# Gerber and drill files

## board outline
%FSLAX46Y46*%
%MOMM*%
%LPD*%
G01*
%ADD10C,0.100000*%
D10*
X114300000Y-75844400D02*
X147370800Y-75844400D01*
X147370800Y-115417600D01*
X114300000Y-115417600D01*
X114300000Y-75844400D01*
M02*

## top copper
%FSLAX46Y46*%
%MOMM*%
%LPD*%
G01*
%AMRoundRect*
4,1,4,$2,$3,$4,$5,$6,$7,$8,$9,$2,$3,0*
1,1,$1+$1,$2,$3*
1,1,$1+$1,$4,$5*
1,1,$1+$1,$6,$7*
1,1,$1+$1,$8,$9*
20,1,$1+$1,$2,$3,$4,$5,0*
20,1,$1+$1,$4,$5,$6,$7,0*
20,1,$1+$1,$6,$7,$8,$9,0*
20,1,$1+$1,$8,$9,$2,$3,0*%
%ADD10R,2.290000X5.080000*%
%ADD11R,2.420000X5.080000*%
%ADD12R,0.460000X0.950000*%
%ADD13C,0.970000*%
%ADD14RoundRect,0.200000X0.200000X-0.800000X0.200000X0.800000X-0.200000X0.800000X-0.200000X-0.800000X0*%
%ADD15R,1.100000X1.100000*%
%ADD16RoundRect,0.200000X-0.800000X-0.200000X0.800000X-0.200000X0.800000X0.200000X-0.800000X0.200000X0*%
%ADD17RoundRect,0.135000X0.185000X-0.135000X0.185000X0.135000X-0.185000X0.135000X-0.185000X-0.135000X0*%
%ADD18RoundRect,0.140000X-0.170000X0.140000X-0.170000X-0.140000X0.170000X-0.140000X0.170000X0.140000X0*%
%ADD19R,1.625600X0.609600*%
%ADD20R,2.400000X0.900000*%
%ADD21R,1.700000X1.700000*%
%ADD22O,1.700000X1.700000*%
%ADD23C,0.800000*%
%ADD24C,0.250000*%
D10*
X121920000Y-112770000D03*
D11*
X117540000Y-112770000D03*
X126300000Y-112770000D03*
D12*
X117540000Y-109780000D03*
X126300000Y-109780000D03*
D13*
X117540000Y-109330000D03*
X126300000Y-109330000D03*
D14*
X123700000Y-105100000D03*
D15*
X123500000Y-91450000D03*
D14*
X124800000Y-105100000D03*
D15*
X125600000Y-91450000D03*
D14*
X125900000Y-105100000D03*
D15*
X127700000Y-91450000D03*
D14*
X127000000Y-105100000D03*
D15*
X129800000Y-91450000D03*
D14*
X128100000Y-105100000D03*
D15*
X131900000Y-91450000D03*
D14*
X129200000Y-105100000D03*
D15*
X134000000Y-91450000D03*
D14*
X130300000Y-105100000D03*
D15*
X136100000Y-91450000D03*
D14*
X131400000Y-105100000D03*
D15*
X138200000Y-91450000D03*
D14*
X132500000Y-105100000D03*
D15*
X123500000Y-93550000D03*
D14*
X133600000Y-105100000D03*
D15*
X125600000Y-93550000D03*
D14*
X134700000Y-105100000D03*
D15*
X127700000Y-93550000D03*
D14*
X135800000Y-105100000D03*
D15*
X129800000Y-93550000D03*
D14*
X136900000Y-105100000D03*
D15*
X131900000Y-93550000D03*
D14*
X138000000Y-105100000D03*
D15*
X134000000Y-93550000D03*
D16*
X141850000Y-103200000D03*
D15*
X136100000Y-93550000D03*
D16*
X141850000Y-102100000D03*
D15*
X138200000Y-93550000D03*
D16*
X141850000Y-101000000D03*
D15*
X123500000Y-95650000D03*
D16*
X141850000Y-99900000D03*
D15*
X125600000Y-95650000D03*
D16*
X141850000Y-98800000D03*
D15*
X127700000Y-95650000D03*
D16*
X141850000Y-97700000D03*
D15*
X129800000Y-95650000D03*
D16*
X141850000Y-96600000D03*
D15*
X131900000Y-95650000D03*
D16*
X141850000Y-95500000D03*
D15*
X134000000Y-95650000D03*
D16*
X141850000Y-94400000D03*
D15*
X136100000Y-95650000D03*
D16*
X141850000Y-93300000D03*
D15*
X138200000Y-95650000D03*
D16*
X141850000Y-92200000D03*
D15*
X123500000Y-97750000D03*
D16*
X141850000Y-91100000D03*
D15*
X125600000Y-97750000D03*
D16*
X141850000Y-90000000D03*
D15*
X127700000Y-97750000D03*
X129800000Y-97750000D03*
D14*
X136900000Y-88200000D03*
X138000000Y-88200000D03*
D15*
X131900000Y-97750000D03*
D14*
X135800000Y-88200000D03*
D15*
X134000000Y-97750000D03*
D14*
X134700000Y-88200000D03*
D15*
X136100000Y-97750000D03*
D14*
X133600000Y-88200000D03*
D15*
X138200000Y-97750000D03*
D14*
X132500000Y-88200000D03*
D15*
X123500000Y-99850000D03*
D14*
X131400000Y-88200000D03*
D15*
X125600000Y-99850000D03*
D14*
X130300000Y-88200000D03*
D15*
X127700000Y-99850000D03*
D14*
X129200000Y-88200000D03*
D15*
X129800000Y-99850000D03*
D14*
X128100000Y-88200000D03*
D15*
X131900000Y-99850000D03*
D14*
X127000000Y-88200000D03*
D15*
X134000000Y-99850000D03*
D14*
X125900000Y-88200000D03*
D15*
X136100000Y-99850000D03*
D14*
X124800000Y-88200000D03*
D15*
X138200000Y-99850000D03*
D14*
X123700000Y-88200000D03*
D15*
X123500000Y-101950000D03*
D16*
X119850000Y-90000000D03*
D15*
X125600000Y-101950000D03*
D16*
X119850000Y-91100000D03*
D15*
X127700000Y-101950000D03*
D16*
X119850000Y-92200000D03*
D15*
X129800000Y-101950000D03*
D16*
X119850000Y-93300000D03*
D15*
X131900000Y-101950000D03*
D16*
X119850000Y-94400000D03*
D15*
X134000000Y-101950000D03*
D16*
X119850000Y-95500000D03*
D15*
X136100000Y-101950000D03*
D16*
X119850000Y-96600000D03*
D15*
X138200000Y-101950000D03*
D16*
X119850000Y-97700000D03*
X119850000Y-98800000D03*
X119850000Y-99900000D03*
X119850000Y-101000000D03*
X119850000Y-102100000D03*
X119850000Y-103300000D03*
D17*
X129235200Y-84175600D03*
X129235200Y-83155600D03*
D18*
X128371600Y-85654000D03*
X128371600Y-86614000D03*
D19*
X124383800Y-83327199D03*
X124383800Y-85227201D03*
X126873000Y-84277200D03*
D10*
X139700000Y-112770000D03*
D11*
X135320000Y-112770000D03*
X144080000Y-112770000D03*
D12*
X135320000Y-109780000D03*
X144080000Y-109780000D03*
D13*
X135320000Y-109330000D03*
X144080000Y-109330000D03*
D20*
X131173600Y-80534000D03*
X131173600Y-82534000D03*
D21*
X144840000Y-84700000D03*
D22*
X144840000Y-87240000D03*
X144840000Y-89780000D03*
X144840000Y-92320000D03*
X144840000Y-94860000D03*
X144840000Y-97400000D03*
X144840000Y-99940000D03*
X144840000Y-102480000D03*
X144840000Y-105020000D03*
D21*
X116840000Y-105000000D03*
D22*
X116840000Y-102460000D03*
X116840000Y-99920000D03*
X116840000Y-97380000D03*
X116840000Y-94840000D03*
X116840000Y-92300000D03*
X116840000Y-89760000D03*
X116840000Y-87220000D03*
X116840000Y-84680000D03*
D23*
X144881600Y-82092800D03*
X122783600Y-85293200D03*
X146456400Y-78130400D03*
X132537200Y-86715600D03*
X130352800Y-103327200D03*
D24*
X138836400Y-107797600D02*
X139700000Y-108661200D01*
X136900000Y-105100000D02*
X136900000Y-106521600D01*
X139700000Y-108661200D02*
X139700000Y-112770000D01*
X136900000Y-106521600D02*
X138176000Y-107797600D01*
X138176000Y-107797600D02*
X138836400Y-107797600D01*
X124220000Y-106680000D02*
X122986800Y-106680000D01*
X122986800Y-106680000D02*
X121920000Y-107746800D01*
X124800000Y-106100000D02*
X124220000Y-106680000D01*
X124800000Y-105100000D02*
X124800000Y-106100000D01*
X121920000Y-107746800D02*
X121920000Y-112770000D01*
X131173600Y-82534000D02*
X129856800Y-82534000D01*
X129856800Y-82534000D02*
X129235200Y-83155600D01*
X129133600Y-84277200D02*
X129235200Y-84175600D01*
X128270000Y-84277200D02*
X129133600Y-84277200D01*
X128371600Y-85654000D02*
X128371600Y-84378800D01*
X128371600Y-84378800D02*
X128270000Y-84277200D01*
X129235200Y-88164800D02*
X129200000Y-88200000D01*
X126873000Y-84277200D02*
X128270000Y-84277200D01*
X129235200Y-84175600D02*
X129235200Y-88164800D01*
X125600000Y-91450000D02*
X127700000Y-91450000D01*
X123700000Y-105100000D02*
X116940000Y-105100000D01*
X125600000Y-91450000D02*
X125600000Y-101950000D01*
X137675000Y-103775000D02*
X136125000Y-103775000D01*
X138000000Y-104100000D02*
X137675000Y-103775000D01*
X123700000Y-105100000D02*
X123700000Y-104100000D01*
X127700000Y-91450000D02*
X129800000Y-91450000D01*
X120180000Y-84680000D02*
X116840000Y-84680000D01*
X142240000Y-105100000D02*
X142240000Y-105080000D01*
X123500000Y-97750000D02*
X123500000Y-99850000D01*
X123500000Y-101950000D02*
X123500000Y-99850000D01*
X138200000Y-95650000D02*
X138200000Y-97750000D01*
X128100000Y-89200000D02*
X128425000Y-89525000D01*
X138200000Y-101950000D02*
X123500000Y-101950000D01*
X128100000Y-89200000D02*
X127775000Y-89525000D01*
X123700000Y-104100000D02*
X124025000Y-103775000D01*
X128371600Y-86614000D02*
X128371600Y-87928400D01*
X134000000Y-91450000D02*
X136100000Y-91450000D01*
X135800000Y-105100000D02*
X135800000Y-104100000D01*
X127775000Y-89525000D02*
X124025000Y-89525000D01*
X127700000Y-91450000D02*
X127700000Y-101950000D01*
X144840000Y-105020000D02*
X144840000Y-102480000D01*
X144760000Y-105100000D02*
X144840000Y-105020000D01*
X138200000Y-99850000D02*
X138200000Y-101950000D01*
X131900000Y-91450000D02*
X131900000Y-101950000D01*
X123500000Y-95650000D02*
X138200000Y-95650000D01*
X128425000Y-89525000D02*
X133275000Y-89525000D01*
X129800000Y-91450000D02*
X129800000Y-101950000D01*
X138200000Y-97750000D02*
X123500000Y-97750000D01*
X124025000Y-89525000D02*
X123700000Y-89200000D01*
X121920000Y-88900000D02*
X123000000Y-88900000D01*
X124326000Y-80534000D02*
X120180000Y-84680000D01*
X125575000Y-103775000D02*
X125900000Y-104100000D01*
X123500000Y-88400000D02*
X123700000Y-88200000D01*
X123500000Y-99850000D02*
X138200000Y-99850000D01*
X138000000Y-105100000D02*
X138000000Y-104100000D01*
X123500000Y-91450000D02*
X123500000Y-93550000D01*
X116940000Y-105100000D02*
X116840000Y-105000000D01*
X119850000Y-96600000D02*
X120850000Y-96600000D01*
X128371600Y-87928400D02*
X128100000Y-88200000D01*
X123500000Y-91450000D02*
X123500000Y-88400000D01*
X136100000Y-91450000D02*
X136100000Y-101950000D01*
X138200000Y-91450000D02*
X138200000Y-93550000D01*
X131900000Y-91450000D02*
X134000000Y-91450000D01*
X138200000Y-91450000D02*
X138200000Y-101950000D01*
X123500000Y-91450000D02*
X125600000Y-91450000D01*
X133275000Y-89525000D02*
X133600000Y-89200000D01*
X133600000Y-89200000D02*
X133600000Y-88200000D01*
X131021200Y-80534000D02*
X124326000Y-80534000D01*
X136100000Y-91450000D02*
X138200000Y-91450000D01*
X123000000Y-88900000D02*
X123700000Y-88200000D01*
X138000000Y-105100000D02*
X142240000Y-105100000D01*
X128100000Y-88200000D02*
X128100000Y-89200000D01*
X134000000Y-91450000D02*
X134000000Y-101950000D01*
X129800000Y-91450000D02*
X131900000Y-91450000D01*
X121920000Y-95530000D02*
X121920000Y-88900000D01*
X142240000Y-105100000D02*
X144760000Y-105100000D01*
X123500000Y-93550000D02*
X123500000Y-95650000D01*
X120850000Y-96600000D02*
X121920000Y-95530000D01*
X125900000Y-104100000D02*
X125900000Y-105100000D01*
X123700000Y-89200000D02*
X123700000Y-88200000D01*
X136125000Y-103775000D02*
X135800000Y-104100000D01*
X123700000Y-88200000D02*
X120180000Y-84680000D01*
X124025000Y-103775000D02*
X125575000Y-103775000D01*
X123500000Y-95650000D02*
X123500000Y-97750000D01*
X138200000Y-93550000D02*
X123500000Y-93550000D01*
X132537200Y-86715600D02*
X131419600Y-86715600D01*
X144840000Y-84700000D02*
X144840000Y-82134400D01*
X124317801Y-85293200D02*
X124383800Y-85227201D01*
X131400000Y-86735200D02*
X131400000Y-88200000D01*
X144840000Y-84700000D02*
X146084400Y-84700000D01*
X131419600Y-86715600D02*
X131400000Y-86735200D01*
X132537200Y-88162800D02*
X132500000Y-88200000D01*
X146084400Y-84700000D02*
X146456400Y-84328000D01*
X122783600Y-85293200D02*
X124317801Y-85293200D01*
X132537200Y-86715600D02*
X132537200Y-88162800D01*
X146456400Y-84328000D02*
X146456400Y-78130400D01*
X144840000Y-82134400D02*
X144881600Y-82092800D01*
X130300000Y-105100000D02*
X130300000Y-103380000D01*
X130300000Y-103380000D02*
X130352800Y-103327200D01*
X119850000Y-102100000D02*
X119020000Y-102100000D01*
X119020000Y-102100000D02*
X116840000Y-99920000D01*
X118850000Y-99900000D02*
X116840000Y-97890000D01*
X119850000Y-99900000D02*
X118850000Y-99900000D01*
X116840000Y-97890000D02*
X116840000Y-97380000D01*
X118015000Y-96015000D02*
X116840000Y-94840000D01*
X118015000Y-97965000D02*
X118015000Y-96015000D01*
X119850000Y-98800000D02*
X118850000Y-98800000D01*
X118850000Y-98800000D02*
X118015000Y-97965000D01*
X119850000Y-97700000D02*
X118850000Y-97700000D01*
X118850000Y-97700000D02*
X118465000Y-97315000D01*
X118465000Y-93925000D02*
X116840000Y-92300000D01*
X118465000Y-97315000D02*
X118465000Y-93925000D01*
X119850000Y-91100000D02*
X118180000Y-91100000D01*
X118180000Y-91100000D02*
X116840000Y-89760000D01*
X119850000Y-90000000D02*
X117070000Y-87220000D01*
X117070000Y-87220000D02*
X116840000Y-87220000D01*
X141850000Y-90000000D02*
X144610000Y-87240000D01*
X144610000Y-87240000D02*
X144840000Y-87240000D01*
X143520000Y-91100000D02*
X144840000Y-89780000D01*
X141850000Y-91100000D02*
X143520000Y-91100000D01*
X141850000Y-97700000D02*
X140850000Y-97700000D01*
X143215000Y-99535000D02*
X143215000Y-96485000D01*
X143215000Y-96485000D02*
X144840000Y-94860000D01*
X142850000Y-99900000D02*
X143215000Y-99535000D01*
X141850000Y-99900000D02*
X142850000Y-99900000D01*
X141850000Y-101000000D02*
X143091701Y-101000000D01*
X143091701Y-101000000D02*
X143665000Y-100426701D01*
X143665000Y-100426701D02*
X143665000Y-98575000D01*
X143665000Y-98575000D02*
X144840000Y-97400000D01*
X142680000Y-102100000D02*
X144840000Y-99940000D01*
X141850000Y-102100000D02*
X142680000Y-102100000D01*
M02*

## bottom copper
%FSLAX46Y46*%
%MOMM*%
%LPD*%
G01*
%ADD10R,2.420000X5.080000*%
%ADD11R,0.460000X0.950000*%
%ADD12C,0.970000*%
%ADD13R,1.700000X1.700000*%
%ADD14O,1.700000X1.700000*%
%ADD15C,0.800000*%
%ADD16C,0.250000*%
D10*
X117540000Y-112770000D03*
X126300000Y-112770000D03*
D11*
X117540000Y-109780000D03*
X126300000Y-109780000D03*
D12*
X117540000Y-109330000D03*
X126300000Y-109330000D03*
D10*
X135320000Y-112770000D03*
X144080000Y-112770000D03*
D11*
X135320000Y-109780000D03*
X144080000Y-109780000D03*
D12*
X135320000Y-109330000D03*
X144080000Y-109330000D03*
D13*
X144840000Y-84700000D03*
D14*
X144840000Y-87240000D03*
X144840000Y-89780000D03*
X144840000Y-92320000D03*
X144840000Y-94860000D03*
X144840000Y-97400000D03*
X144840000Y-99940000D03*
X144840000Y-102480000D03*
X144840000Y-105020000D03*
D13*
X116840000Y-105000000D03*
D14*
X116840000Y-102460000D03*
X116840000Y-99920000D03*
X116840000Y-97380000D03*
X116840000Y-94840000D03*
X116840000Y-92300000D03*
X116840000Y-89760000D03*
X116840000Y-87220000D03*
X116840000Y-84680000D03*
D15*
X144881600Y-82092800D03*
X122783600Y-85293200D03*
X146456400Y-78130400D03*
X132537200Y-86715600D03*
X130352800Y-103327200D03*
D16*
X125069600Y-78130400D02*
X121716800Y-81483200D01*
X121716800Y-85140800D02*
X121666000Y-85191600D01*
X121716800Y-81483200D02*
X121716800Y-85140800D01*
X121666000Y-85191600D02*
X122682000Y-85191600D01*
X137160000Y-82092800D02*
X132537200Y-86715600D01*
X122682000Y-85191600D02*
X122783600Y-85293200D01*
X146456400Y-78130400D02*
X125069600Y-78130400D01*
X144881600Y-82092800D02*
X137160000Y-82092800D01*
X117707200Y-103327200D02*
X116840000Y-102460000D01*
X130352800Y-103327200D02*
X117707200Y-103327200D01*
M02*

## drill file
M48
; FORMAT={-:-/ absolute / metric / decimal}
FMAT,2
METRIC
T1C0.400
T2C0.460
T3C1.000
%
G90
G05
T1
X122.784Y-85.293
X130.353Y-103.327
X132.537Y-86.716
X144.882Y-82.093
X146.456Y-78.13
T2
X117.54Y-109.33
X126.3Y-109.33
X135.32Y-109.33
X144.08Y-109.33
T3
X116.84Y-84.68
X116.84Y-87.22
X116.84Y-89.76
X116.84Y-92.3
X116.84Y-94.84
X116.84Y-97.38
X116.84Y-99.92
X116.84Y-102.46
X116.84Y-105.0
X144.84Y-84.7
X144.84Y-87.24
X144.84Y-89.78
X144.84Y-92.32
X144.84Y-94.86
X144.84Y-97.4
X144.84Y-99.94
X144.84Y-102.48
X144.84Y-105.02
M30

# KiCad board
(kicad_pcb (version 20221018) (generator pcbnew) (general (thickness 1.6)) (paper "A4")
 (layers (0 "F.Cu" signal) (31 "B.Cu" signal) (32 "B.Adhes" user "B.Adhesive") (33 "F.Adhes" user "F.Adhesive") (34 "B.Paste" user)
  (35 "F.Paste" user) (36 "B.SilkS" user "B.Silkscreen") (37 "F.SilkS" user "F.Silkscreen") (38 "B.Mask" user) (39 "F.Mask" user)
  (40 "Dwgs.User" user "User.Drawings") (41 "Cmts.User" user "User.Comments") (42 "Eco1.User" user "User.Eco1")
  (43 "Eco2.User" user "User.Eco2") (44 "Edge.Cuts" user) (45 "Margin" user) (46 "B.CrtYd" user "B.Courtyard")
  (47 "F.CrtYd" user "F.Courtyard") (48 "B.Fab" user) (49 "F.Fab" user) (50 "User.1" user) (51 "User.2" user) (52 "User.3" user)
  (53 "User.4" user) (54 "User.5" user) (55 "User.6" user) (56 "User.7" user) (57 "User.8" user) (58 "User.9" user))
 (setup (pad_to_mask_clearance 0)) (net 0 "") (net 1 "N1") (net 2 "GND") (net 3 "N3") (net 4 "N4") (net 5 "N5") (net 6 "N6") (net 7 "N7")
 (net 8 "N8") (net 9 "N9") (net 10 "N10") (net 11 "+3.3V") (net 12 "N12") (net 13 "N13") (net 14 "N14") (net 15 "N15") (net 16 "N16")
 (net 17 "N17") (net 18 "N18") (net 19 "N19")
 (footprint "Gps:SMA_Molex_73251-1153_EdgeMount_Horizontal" (layer "F.Cu") (at 121.92 111.05 90)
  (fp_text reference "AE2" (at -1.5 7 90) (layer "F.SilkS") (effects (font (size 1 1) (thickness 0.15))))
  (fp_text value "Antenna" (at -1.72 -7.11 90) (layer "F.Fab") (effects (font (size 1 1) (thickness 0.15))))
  (pad "1" smd rect (at -1.72 0 90) (size 5.08 2.29) (layers "F.Cu" "F.Paste" "F.Mask") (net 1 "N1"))
  (pad "2" smd rect (at -1.72 -4.38 90) (size 5.08 2.42) (layers "F.Cu" "F.Paste" "F.Mask"))
  (pad "2" smd rect (at -1.72 -4.38 90) (size 5.08 2.42) (layers "B.Cu" "B.Paste" "B.Mask"))
  (pad "2" smd rect (at -1.72 4.38 90) (size 5.08 2.42) (layers "F.Cu" "F.Paste" "F.Mask"))
  (pad "2" smd rect (at -1.72 4.38 90) (size 5.08 2.42) (layers "B.Cu" "B.Paste" "B.Mask"))
  (pad "2" smd rect (at 1.27 -4.38 90) (size 0.95 0.46) (layers "F.Cu"))
  (pad "2" smd rect (at 1.27 -4.38 90) (size 0.95 0.46) (layers "B.Cu"))
  (pad "2" smd rect (at 1.27 4.38 90) (size 0.95 0.46) (layers "F.Cu"))
  (pad "2" smd rect (at 1.27 4.38 90) (size 0.95 0.46) (layers "B.Cu"))
  (pad "2" thru_hole circle (at 1.72 -4.38 90) (size 0.97 0.97) (drill 0.46) (layers "*.Cu"))
  (pad "2" thru_hole circle (at 1.72 4.38 90) (size 0.97 0.97) (drill 0.46) (layers "*.Cu")))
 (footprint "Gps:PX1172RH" (layer "F.Cu") (at 119.85 90)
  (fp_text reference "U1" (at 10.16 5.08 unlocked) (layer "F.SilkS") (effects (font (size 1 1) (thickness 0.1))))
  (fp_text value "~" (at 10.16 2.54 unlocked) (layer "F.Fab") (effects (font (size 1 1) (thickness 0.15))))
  (pad "1" smd roundrect (at 3.85 15.1 90) (size 2 0.8) (layers "F.Cu" "F.Paste" "F.Mask") (roundrect_rratio 0.25) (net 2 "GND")
   (thermal_bridge_angle 45))
  (pad "1$" smd rect (at 3.65 1.45) (size 1.1 1.1) (layers "F.Cu" "F.Paste" "F.Mask") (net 2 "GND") (thermal_bridge_angle 45))
  (pad "2" smd roundrect (at 4.95 15.1 90) (size 2 0.8) (layers "F.Cu" "F.Paste" "F.Mask") (roundrect_rratio 0.25) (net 1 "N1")
   (thermal_bridge_angle 45))
  (pad "2$" smd rect (at 5.75 1.45) (size 1.1 1.1) (layers "F.Cu" "F.Paste" "F.Mask") (thermal_bridge_angle 45))
  (pad "3" smd roundrect (at 6.05 15.1 90) (size 2 0.8) (layers "F.Cu" "F.Paste" "F.Mask") (roundrect_rratio 0.25) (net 2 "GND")
   (thermal_bridge_angle 45))
  (pad "3$" smd rect (at 7.85 1.45) (size 1.1 1.1) (layers "F.Cu" "F.Paste" "F.Mask") (thermal_bridge_angle 45))
  (pad "4" smd roundrect (at 7.15 15.1 90) (size 2 0.8) (layers "F.Cu" "F.Paste" "F.Mask") (roundrect_rratio 0.25) (thermal_bridge_angle 45))
  (pad "4$" smd rect (at 9.95 1.45) (size 1.1 1.1) (layers "F.Cu" "F.Paste" "F.Mask") (thermal_bridge_angle 45))
  (pad "5" smd roundrect (at 8.25 15.1 90) (size 2 0.8) (layers "F.Cu" "F.Paste" "F.Mask") (roundrect_rratio 0.25) (thermal_bridge_angle 45))
  (pad "5$" smd rect (at 12.05 1.45) (size 1.1 1.1) (layers "F.Cu" "F.Paste" "F.Mask") (thermal_bridge_angle 45))
  (pad "6" smd roundrect (at 9.35 15.1 90) (size 2 0.8) (layers "F.Cu" "F.Paste" "F.Mask") (roundrect_rratio 0.25) (thermal_bridge_angle 45))
  (pad "6$" smd rect (at 14.15 1.45) (size 1.1 1.1) (layers "F.Cu" "F.Paste" "F.Mask") (thermal_bridge_angle 45))
  (pad "7" smd roundrect (at 10.45 15.1 90) (size 2 0.8) (layers "F.Cu" "F.Paste" "F.Mask") (roundrect_rratio 0.25) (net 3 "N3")
   (thermal_bridge_angle 45))
  (pad "7$" smd rect (at 16.25 1.45) (size 1.1 1.1) (layers "F.Cu" "F.Paste" "F.Mask") (thermal_bridge_angle 45))
  (pad "8" smd roundrect (at 11.55 15.1 90) (size 2 0.8) (layers "F.Cu" "F.Paste" "F.Mask") (roundrect_rratio 0.25)
   (thermal_bridge_angle 45))
  (pad "8$" smd rect (at 18.35 1.45) (size 1.1 1.1) (layers "F.Cu" "F.Paste" "F.Mask") (thermal_bridge_angle 45))
  (pad "9" smd roundrect (at 12.65 15.1 90) (size 2 0.8) (layers "F.Cu" "F.Paste" "F.Mask") (roundrect_rratio 0.25)
   (thermal_bridge_angle 45))
  (pad "9$" smd rect (at 3.65 3.55) (size 1.1 1.1) (layers "F.Cu" "F.Paste" "F.Mask") (thermal_bridge_angle 45))
  (pad "10" smd roundrect (at 13.75 15.1 90) (size 2 0.8) (layers "F.Cu" "F.Paste" "F.Mask") (roundrect_rratio 0.25)
   (thermal_bridge_angle 45))
  (pad "10$" smd rect (at 5.75 3.55) (size 1.1 1.1) (layers "F.Cu" "F.Paste" "F.Mask") (thermal_bridge_angle 45))
  (pad "11" smd roundrect (at 14.85 15.1 90) (size 2 0.8) (layers "F.Cu" "F.Paste" "F.Mask") (roundrect_rratio 0.25)
   (thermal_bridge_angle 45))
  (pad "11$" smd rect (at 7.85 3.55) (size 1.1 1.1) (layers "F.Cu" "F.Paste" "F.Mask") (thermal_bridge_angle 45))
  (pad "12" smd roundrect (at 15.95 15.1 90) (size 2 0.8) (layers "F.Cu" "F.Paste" "F.Mask") (roundrect_rratio 0.25) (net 2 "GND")
   (thermal_bridge_angle 45))
  (pad "12$" smd rect (at 9.95 3.55) (size 1.1 1.1) (layers "F.Cu" "F.Paste" "F.Mask") (thermal_bridge_angle 45))
  (pad "13" smd roundrect (at 17.05 15.1 90) (size 2 0.8) (layers "F.Cu" "F.Paste" "F.Mask") (roundrect_rratio 0.25) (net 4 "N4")
   (thermal_bridge_angle 45))
  (pad "13$" smd rect (at 12.05 3.55) (size 1.1 1.1) (layers "F.Cu" "F.Paste" "F.Mask") (thermal_bridge_angle 45))
  (pad "14" smd roundrect (at 18.15 15.1 90) (size 2 0.8) (layers "F.Cu" "F.Paste" "F.Mask") (roundrect_rratio 0.25) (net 2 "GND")
   (thermal_bridge_angle 45))
  (pad "14$" smd rect (at 14.15 3.55) (size 1.1 1.1) (layers "F.Cu" "F.Paste" "F.Mask") (thermal_bridge_angle 45))
  (pad "15" smd roundrect (at 22 13.2) (size 2 0.8) (layers "F.Cu" "F.Paste" "F.Mask") (roundrect_rratio 0.25) (thermal_bridge_angle 45))
  (pad "15$" smd rect (at 16.25 3.55) (size 1.1 1.1) (layers "F.Cu" "F.Paste" "F.Mask") (thermal_bridge_angle 45))
  (pad "16" smd roundrect (at 22 12.1) (size 2 0.8) (layers "F.Cu" "F.Paste" "F.Mask") (roundrect_rratio 0.25) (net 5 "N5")
   (thermal_bridge_angle 45))
  (pad "16$" smd rect (at 18.35 3.55) (size 1.1 1.1) (layers "F.Cu" "F.Paste" "F.Mask") (thermal_bridge_angle 45))
  (pad "17" smd roundrect (at 22 11) (size 2 0.8) (layers "F.Cu" "F.Paste" "F.Mask") (roundrect_rratio 0.25) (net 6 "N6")
   (thermal_bridge_angle 45))
  (pad "17$" smd rect (at 3.65 5.65) (size 1.1 1.1) (layers "F.Cu" "F.Paste" "F.Mask") (thermal_bridge_angle 45))
  (pad "18" smd roundrect (at 22 9.9) (size 2 0.8) (layers "F.Cu" "F.Paste" "F.Mask") (roundrect_rratio 0.25) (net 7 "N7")
   (thermal_bridge_angle 45))
  (pad "18$" smd rect (at 5.75 5.65) (size 1.1 1.1) (layers "F.Cu" "F.Paste" "F.Mask") (thermal_bridge_angle 45))
  (pad "19" smd roundrect (at 22 8.8) (size 2 0.8) (layers "F.Cu" "F.Paste" "F.Mask") (roundrect_rratio 0.25) (thermal_bridge_angle 45))
  (pad "19$" smd rect (at 7.85 5.65) (size 1.1 1.1) (layers "F.Cu" "F.Paste" "F.Mask") (thermal_bridge_angle 45))
  (pad "20" smd roundrect (at 22 7.7) (size 2 0.8) (layers "F.Cu" "F.Paste" "F.Mask") (roundrect_rratio 0.25) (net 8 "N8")
   (thermal_bridge_angle 45))
  (pad "20$" smd rect (at 9.95 5.65) (size 1.1 1.1) (layers "F.Cu" "F.Paste" "F.Mask") (thermal_bridge_angle 45))
  (pad "21" smd roundrect (at 22 6.6) (size 2 0.8) (layers "F.Cu" "F.Paste" "F.Mask") (roundrect_rratio 0.25) (thermal_bridge_angle 45))
  (pad "21$" smd rect (at 12.05 5.65) (size 1.1 1.1) (layers "F.Cu" "F.Paste" "F.Mask") (thermal_bridge_angle 45))
  (pad "22" smd roundrect (at 22 5.5) (size 2 0.8) (layers "F.Cu" "F.Paste" "F.Mask") (roundrect_rratio 0.25) (thermal_bridge_angle 45))
  (pad "22$" smd rect (at 14.15 5.65) (size 1.1 1.1) (layers "F.Cu" "F.Paste" "F.Mask") (thermal_bridge_angle 45))
  (pad "23" smd roundrect (at 22 4.4) (size 2 0.8) (layers "F.Cu" "F.Paste" "F.Mask") (roundrect_rratio 0.25) (thermal_bridge_angle 45))
  (pad "23$" smd rect (at 16.25 5.65) (size 1.1 1.1) (layers "F.Cu" "F.Paste" "F.Mask") (thermal_bridge_angle 45))
  (pad "24" smd roundrect (at 22 3.3) (size 2 0.8) (layers "F.Cu" "F.Paste" "F.Mask") (roundrect_rratio 0.25) (thermal_bridge_angle 45))
  (pad "24$" smd rect (at 18.35 5.65) (size 1.1 1.1) (layers "F.Cu" "F.Paste" "F.Mask") (thermal_bridge_angle 45))
  (pad "25" smd roundrect (at 22 2.2) (size 2 0.8) (layers "F.Cu" "F.Mask") (roundrect_rratio 0.25) (thermal_bridge_angle 45))
  (pad "25$" smd rect (at 3.65 7.75) (size 1.1 1.1) (layers "F.Cu" "F.Paste" "F.Mask") (thermal_bridge_angle 45))
  (pad "26" smd roundrect (at 22 1.1) (size 2 0.8) (layers "F.Cu" "F.Paste" "F.Mask") (roundrect_rratio 0.25) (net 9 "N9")
   (thermal_bridge_angle 45))
  (pad "26$" smd rect (at 5.75 7.75) (size 1.1 1.1) (layers "F.Cu" "F.Paste" "F.Mask") (thermal_bridge_angle 45))
  (pad "27" smd roundrect (at 22 0) (size 2 0.8) (layers "F.Cu" "F.Paste" "F.Mask") (roundrect_rratio 0.25) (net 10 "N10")
   (thermal_bridge_angle 45))
  (pad "27$" smd rect (at 7.85 7.75) (size 1.1 1.1) (layers "F.Cu" "F.Paste" "F.Mask") (thermal_bridge_angle 45))
  (pad "28$" smd rect (at 9.95 7.75) (size 1.1 1.1) (layers "F.Cu" "F.Paste" "F.Mask") (thermal_bridge_angle 45))
  (pad "29" smd roundrect (at 17.05 -1.8 90) (size 2 0.8) (layers "F.Cu" "F.Paste" "F.Mask") (roundrect_rratio 0.25)
   (thermal_bridge_angle 45))
  (pad "29" smd roundrect (at 18.15 -1.8 90) (size 2 0.8) (layers "F.Cu" "F.Paste" "F.Mask") (roundrect_rratio 0.25)
   (thermal_bridge_angle 45))
  (pad "29$" smd rect (at 12.05 7.75) (size 1.1 1.1) (layers "F.Cu" "F.Paste" "F.Mask") (thermal_bridge_angle 45))
  (pad "30" smd roundrect (at 15.95 -1.8 90) (size 2 0.8) (layers "F.Cu" "F.Paste" "F.Mask") (roundrect_rratio 0.25)
   (thermal_bridge_angle 45))
  (pad "30$" smd rect (at 14.15 7.75) (size 1.1 1.1) (layers "F.Cu" "F.Paste" "F.Mask") (thermal_bridge_angle 45))
  (pad "31" smd roundrect (at 14.85 -1.8 90) (size 2 0.8) (layers "F.Cu" "F.Paste" "F.Mask") (roundrect_rratio 0.25)
   (thermal_bridge_angle 45))
  (pad "31$" smd rect (at 16.25 7.75) (size 1.1 1.1) (layers "F.Cu" "F.Paste" "F.Mask") (thermal_bridge_angle 45))
  (pad "32" smd roundrect (at 13.75 -1.8 90) (size 2 0.8) (layers "F.Cu" "F.Paste" "F.Mask") (roundrect_rratio 0.25) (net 2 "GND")
   (thermal_bridge_angle 45))
  (pad "32$" smd rect (at 18.35 7.75) (size 1.1 1.1) (layers "F.Cu" "F.Paste" "F.Mask") (thermal_bridge_angle 45))
  (pad "33" smd roundrect (at 12.65 -1.8 90) (size 2 0.8) (layers "F.Cu" "F.Paste" "F.Mask") (roundrect_rratio 0.25) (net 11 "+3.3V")
   (thermal_bridge_angle 45))
  (pad "33$" smd rect (at 3.65 9.85) (size 1.1 1.1) (layers "F.Cu" "F.Paste" "F.Mask") (thermal_bridge_angle 45))
  (pad "34" smd roundrect (at 11.55 -1.8 90) (size 2 0.8) (layers "F.Cu" "F.Paste" "F.Mask") (roundrect_rratio 0.25) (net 11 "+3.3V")
   (thermal_bridge_angle 45))
  (pad "34$" smd rect (at 5.75 9.85) (size 1.1 1.1) (layers "F.Cu" "F.Paste" "F.Mask") (thermal_bridge_angle 45))
  (pad "35" smd roundrect (at 10.45 -1.8 90) (size 2 0.8) (layers "F.Cu" "F.Paste" "F.Mask") (roundrect_rratio 0.25)
   (thermal_bridge_angle 45))
  (pad "35$" smd rect (at 7.85 9.85) (size 1.1 1.1) (layers "F.Cu" "F.Paste" "F.Mask") (thermal_bridge_angle 45))
  (pad "36" smd roundrect (at 9.35 -1.8 90) (size 2 0.8) (layers "F.Cu" "F.Paste" "F.Mask") (roundrect_rratio 0.25) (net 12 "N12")
   (thermal_bridge_angle 45))
  (pad "36$" smd rect (at 9.95 9.85) (size 1.1 1.1) (layers "F.Cu" "F.Paste" "F.Mask") (thermal_bridge_angle 45))
  (pad "37" smd roundrect (at 8.25 -1.8 90) (size 2 0.8) (layers "F.Cu" "F.Paste" "F.Mask") (roundrect_rratio 0.25) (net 2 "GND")
   (thermal_bridge_angle 45))
  (pad "37$" smd rect (at 12.05 9.85) (size 1.1 1.1) (layers "F.Cu" "F.Paste" "F.Mask") (thermal_bridge_angle 45))
  (pad "38" smd roundrect (at 7.15 -1.8 90) (size 2 0.8) (layers "F.Cu" "F.Paste" "F.Mask") (roundrect_rratio 0.25)
   (thermal_bridge_angle 45))
  (pad "38$" smd rect (at 14.15 9.85) (size 1.1 1.1) (layers "F.Cu" "F.Paste" "F.Mask") (thermal_bridge_angle 45))
  (pad "39" smd roundrect (at 6.05 -1.8 90) (size 2 0.8) (layers "F.Cu" "F.Paste" "F.Mask") (roundrect_rratio 0.25)
   (thermal_bridge_angle 45))
  (pad "39$" smd rect (at 16.25 9.85) (size 1.1 1.1) (layers "F.Cu" "F.Paste" "F.Mask") (thermal_bridge_angle 45))
  (pad "40" smd roundrect (at 4.95 -1.8 90) (size 2 0.8) (layers "F.Cu" "F.Paste" "F.Mask") (roundrect_rratio 0.25)
   (thermal_bridge_angle 45))
  (pad "40$" smd rect (at 18.35 9.85) (size 1.1 1.1) (layers "F.Cu" "F.Paste" "F.Mask") (thermal_bridge_angle 45))
  (pad "41" smd roundrect (at 3.85 -1.8 90) (size 2 0.8) (layers "F.Cu" "F.Paste" "F.Mask") (roundrect_rratio 0.25) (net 2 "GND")
   (thermal_bridge_angle 45))
  (pad "41$" smd rect (at 3.65 11.95) (size 1.1 1.1) (layers "F.Cu" "F.Paste" "F.Mask") (thermal_bridge_angle 45))
  (pad "42" smd roundrect (at 0 0) (size 2 0.8) (layers "F.Cu" "F.Paste" "F.Mask") (roundrect_rratio 0.25) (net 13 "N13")
   (thermal_bridge_angle 45))
  (pad "42$" smd rect (at 5.75 11.95) (size 1.1 1.1) (layers "F.Cu" "F.Paste" "F.Mask") (thermal_bridge_angle 45))
  (pad "43" smd roundrect (at 0 1.1) (size 2 0.8) (layers "F.Cu" "F.Paste" "F.Mask") (roundrect_rratio 0.25) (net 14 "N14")
   (thermal_bridge_angle 45))
  (pad "43$" smd rect (at 7.85 11.95) (size 1.1 1.1) (layers "F.Cu" "F.Paste" "F.Mask") (thermal_bridge_angle 45))
  (pad "44" smd roundrect (at 0 2.2) (size 2 0.8) (layers "F.Cu" "F.Paste" "F.Mask") (roundrect_rratio 0.25) (thermal_bridge_angle 45))
  (pad "44$" smd rect (at 9.95 11.95) (size 1.1 1.1) (layers "F.Cu" "F.Paste" "F.Mask") (thermal_bridge_angle 45))
  (pad "45" smd roundrect (at 0 3.3) (size 2 0.8) (layers "F.Cu" "F.Paste" "F.Mask") (roundrect_rratio 0.25) (thermal_bridge_angle 45))
  (pad "45$" smd rect (at 12.05 11.95) (size 1.1 1.1) (layers "F.Cu" "F.Paste" "F.Mask") (thermal_bridge_angle 45))
  (pad "46" smd roundrect (at 0 4.4) (size 2 0.8) (layers "F.Cu" "F.Paste" "F.Mask") (roundrect_rratio 0.25) (thermal_bridge_angle 45))
  (pad "46$" smd rect (at 14.15 11.95) (size 1.1 1.1) (layers "F.Cu" "F.Paste" "F.Mask") (thermal_bridge_angle 45))
  (pad "47" smd roundrect (at 0 5.5) (size 2 0.8) (layers "F.Cu" "F.Paste" "F.Mask") (roundrect_rratio 0.25) (thermal_bridge_angle 45))
  (pad "47$" smd rect (at 16.25 11.95) (size 1.1 1.1) (layers "F.Cu" "F.Paste" "F.Mask") (thermal_bridge_angle 45))
  (pad "48" smd roundrect (at 0 6.6) (size 2 0.8) (layers "F.Cu" "F.Paste" "F.Mask") (roundrect_rratio 0.25) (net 2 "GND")
   (thermal_bridge_angle 45))
  (pad "48$" smd rect (at 18.35 11.95) (size 1.1 1.1) (layers "F.Cu" "F.Paste" "F.Mask") (thermal_bridge_angle 45))
  (pad "49" smd roundrect (at 0 7.7) (size 2 0.8) (layers "F.Cu" "F.Paste" "F.Mask") (roundrect_rratio 0.25) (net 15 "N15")
   (thermal_bridge_angle 45))
  (pad "50" smd roundrect (at 0 8.8) (size 2 0.8) (layers "F.Cu" "F.Paste" "F.Mask") (roundrect_rratio 0.25) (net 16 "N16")
   (thermal_bridge_angle 45))
  (pad "51" smd roundrect (at 0 9.9) (size 2 0.8) (layers "F.Cu" "F.Paste" "F.Mask") (roundrect_rratio 0.25) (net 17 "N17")
   (thermal_bridge_angle 45))
  (pad "52" smd roundrect (at 0 11) (size 2 0.8) (layers "F.Cu" "F.Paste" "F.Mask") (roundrect_rratio 0.25) (thermal_bridge_angle 45))
  (pad "53" smd roundrect (at 0 12.1) (size 2 0.8) (layers "F.Cu" "F.Paste" "F.Mask") (roundrect_rratio 0.25) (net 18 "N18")
   (thermal_bridge_angle 45))
  (pad "54" smd roundrect (at 0 13.3) (size 2 0.8) (layers "F.Cu" "F.Paste" "F.Mask") (roundrect_rratio 0.25) (thermal_bridge_angle 45)))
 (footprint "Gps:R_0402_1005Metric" (layer "F.Cu") (at 129.2352 83.6656 90)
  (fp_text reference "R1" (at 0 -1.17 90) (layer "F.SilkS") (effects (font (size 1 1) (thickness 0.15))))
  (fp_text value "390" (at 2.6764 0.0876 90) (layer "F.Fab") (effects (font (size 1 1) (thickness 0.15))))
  (pad "1" smd roundrect (at -0.51 0 90) (size 0.54 0.64) (layers "F.Cu" "F.Paste" "F.Mask") (roundrect_rratio 0.25) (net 12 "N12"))
  (pad "2" smd roundrect (at 0.51 0 90) (size 0.54 0.64) (layers "F.Cu" "F.Paste" "F.Mask") (roundrect_rratio 0.25) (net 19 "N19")))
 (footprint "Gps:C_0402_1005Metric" (layer "F.Cu") (at 128.3716 86.134 -90)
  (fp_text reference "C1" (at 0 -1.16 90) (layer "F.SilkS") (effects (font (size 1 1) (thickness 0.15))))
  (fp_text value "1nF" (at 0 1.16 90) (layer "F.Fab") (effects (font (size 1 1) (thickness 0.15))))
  (pad "1" smd roundrect (at -0.48 0 270) (size 0.56 0.62) (layers "F.Cu" "F.Paste" "F.Mask") (roundrect_rratio 0.25) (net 12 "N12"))
  (pad "2" smd roundrect (at 0.48 0 270) (size 0.56 0.62) (layers "F.Cu" "F.Paste" "F.Mask") (roundrect_rratio 0.25) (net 2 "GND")))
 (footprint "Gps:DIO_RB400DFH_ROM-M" (layer "F.Cu") (at 125.6284 84.2772 -90)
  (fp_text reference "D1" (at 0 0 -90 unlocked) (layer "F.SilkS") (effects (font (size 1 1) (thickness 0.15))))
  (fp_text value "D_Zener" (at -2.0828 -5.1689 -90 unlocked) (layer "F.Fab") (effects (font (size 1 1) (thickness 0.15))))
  (pad "1" smd rect (at -0.950001 1.2446 270) (size 0.6096 1.6256) (layers "F.Cu" "F.Paste" "F.Mask"))
  (pad "2" smd rect (at 0.950001 1.2446 270) (size 0.6096 1.6256) (layers "F.Cu" "F.Paste" "F.Mask") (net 11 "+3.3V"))
  (pad "3" smd rect (at 0 -1.2446 270) (size 0.6096 1.6256) (layers "F.Cu" "F.Paste" "F.Mask") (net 12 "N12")))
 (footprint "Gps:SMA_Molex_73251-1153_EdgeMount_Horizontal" (layer "F.Cu") (at 139.7 111.05 90)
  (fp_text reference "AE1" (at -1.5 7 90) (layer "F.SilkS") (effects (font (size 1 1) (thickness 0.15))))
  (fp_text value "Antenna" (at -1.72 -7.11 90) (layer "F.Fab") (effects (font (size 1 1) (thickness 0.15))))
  (pad "1" smd rect (at -1.72 0 90) (size 5.08 2.29) (layers "F.Cu" "F.Paste" "F.Mask") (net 4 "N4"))
  (pad "2" smd rect (at -1.72 -4.38 90) (size 5.08 2.42) (layers "F.Cu" "F.Paste" "F.Mask"))
  (pad "2" smd rect (at -1.72 -4.38 90) (size 5.08 2.42) (layers "B.Cu" "B.Paste" "B.Mask"))
  (pad "2" smd rect (at -1.72 4.38 90) (size 5.08 2.42) (layers "F.Cu" "F.Paste" "F.Mask"))
  (pad "2" smd rect (at -1.72 4.38 90) (size 5.08 2.42) (layers "B.Cu" "B.Paste" "B.Mask"))
  (pad "2" smd rect (at 1.27 -4.38 90) (size 0.95 0.46) (layers "F.Cu"))
  (pad "2" smd rect (at 1.27 -4.38 90) (size 0.95 0.46) (layers "B.Cu"))
  (pad "2" smd rect (at 1.27 4.38 90) (size 0.95 0.46) (layers "F.Cu"))
  (pad "2" smd rect (at 1.27 4.38 90) (size 0.95 0.46) (layers "B.Cu"))
  (pad "2" thru_hole circle (at 1.72 -4.38 90) (size 0.97 0.97) (drill 0.46) (layers "*.Cu"))
  (pad "2" thru_hole circle (at 1.72 4.38 90) (size 0.97 0.97) (drill 0.46) (layers "*.Cu")))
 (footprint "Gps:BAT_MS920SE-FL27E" (layer "F.Cu") (at 138.0236 81.534 90)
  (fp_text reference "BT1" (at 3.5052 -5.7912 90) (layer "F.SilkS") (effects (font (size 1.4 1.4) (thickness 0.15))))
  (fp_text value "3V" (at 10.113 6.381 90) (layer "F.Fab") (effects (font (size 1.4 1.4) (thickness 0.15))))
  (pad "N" smd rect (at 1 -6.85 180) (size 2.4 0.9) (layers "F.Cu" "F.Paste" "F.Mask") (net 2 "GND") (solder_mask_margin 0.102))
  (pad "P" smd rect (at -1 -6.85 180) (size 2.4 0.9) (layers "F.Cu" "F.Paste" "F.Mask") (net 19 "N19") (solder_mask_margin 0.102)))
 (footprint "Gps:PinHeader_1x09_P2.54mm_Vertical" (layer "B.Cu") (at 144.84 84.7 180)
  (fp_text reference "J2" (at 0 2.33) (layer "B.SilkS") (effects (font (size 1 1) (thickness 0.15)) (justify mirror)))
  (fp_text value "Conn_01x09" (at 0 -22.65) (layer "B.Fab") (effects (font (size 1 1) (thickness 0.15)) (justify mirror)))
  (pad "1" thru_hole rect (at 0 0 180) (size 1.7 1.7) (drill 1) (layers "*.Cu" "*.Mask") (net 11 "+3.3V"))
  (pad "2" thru_hole oval (at 0 -2.54 180) (size 1.7 1.7) (drill 1) (layers "*.Cu" "*.Mask") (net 10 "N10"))
  (pad "3" thru_hole oval (at 0 -5.08 180) (size 1.7 1.7) (drill 1) (layers "*.Cu" "*.Mask") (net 9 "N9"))
  (pad "4" thru_hole oval (at 0 -7.62 180) (size 1.7 1.7) (drill 1) (layers "*.Cu" "*.Mask") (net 8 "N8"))
  (pad "5" thru_hole oval (at 0 -10.16 180) (size 1.7 1.7) (drill 1) (layers "*.Cu" "*.Mask") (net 7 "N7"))
  (pad "6" thru_hole oval (at 0 -12.7 180) (size 1.7 1.7) (drill 1) (layers "*.Cu" "*.Mask") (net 6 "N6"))
  (pad "7" thru_hole oval (at 0 -15.24 180) (size 1.7 1.7) (drill 1) (layers "*.Cu" "*.Mask") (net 5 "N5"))
  (pad "8" thru_hole oval (at 0 -17.78 180) (size 1.7 1.7) (drill 1) (layers "*.Cu" "*.Mask") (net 2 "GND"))
  (pad "9" thru_hole oval (at 0 -20.32 180) (size 1.7 1.7) (drill 1) (layers "*.Cu" "*.Mask") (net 2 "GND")))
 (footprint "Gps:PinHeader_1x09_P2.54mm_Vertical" (layer "B.Cu") (at 116.84 105)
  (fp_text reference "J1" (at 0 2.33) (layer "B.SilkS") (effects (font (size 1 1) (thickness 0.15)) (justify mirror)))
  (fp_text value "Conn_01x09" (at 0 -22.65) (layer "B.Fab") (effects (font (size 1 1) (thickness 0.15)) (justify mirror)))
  (pad "1" thru_hole rect (at 0 0) (size 1.7 1.7) (drill 1) (layers "*.Cu" "*.Mask") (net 2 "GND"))
  (pad "2" thru_hole oval (at 0 -2.54) (size 1.7 1.7) (drill 1) (layers "*.Cu" "*.Mask") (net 3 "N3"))
  (pad "3" thru_hole oval (at 0 -5.08) (size 1.7 1.7) (drill 1) (layers "*.Cu" "*.Mask") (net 18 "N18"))
  (pad "4" thru_hole oval (at 0 -7.62) (size 1.7 1.7) (drill 1) (layers "*.Cu" "*.Mask") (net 17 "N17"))
  (pad "5" thru_hole oval (at 0 -10.16) (size 1.7 1.7) (drill 1) (layers "*.Cu" "*.Mask") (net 16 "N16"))
  (pad "6" thru_hole oval (at 0 -12.7) (size 1.7 1.7) (drill 1) (layers "*.Cu" "*.Mask") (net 15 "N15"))
  (pad "7" thru_hole oval (at 0 -15.24) (size 1.7 1.7) (drill 1) (layers "*.Cu" "*.Mask") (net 14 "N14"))
  (pad "8" thru_hole oval (at 0 -17.78) (size 1.7 1.7) (drill 1) (layers "*.Cu" "*.Mask") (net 13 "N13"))
  (pad "9" thru_hole oval (at 0 -20.32) (size 1.7 1.7) (drill 1) (layers "*.Cu" "*.Mask") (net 2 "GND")))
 (gr_rect (start 114.3 75.8444) (end 147.3708 115.4176) (stroke (width 0.1) (type default)) (fill none) (layer "Edge.Cuts"))
 (segment (start 138.8364 107.7976) (end 139.7 108.6612) (width 0.25) (layer "F.Cu") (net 4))
 (segment (start 136.9 105.1) (end 136.9 106.5216) (width 0.25) (layer "F.Cu") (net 4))
 (segment (start 139.7 108.6612) (end 139.7 112.77) (width 0.25) (layer "F.Cu") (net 4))
 (segment (start 136.9 106.5216) (end 138.176 107.7976) (width 0.25) (layer "F.Cu") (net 4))
 (segment (start 138.176 107.7976) (end 138.8364 107.7976) (width 0.25) (layer "F.Cu") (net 4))
 (segment (start 124.22 106.68) (end 122.9868 106.68) (width 0.25) (layer "F.Cu") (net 1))
 (segment (start 122.9868 106.68) (end 121.92 107.7468) (width 0.25) (layer "F.Cu") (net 1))
 (segment (start 124.8 106.1) (end 124.22 106.68) (width 0.25) (layer "F.Cu") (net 1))
 (segment (start 124.8 105.1) (end 124.8 106.1) (width 0.25) (layer "F.Cu") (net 1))
 (segment (start 121.92 107.7468) (end 121.92 112.77) (width 0.25) (layer "F.Cu") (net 1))
 (segment (start 131.1736 82.534) (end 129.8568 82.534) (width 0.25) (layer "F.Cu") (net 19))
 (segment (start 129.8568 82.534) (end 129.2352 83.1556) (width 0.25) (layer "F.Cu") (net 19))
 (segment (start 129.1336 84.2772) (end 129.2352 84.1756) (width 0.25) (layer "F.Cu") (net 12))
 (segment (start 128.27 84.2772) (end 129.1336 84.2772) (width 0.25) (layer "F.Cu") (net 12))
 (segment (start 128.3716 85.654) (end 128.3716 84.3788) (width 0.25) (layer "F.Cu") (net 12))
 (segment (start 128.3716 84.3788) (end 128.27 84.2772) (width 0.25) (layer "F.Cu") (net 12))
 (segment (start 129.2352 88.1648) (end 129.2 88.2) (width 0.25) (layer "F.Cu") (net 12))
 (segment (start 126.873 84.2772) (end 128.27 84.2772) (width 0.25) (layer "F.Cu") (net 12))
 (segment (start 129.2352 84.1756) (end 129.2352 88.1648) (width 0.25) (layer "F.Cu") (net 12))
 (segment (start 125.6 91.45) (end 127.7 91.45) (width 0.25) (layer "F.Cu") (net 2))
 (segment (start 123.7 105.1) (end 116.94 105.1) (width 0.25) (layer "F.Cu") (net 2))
 (segment (start 125.6 91.45) (end 125.6 101.95) (width 0.25) (layer "F.Cu") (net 2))
 (segment (start 137.675 103.775) (end 136.125 103.775) (width 0.25) (layer "F.Cu") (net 2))
 (segment (start 138 104.1) (end 137.675 103.775) (width 0.25) (layer "F.Cu") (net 2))
 (segment (start 123.7 105.1) (end 123.7 104.1) (width 0.25) (layer "F.Cu") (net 2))
 (segment (start 127.7 91.45) (end 129.8 91.45) (width 0.25) (layer "F.Cu") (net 2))
 (segment (start 120.18 84.68) (end 116.84 84.68) (width 0.25) (layer "F.Cu") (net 2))
 (segment (start 142.24 105.1) (end 142.24 105.08) (width 0.25) (layer "F.Cu") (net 2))
 (segment (start 123.5 97.75) (end 123.5 99.85) (width 0.25) (layer "F.Cu") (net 2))
 (segment (start 123.5 101.95) (end 123.5 99.85) (width 0.25) (layer "F.Cu") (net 2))
 (segment (start 138.2 95.65) (end 138.2 97.75) (width 0.25) (layer "F.Cu") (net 2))
 (segment (start 128.1 89.2) (end 128.425 89.525) (width 0.25) (layer "F.Cu") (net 2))
 (segment (start 138.2 101.95) (end 123.5 101.95) (width 0.25) (layer "F.Cu") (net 2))
 (segment (start 128.1 89.2) (end 127.775 89.525) (width 0.25) (layer "F.Cu") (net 2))
 (segment (start 123.7 104.1) (end 124.025 103.775) (width 0.25) (layer "F.Cu") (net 2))
 (segment (start 128.3716 86.614) (end 128.3716 87.9284) (width 0.25) (layer "F.Cu") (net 2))
 (segment (start 134 91.45) (end 136.1 91.45) (width 0.25) (layer "F.Cu") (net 2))
 (segment (start 135.8 105.1) (end 135.8 104.1) (width 0.25) (layer "F.Cu") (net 2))
 (segment (start 127.775 89.525) (end 124.025 89.525) (width 0.25) (layer "F.Cu") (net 2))
 (segment (start 127.7 91.45) (end 127.7 101.95) (width 0.25) (layer "F.Cu") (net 2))
 (segment (start 144.84 105.02) (end 144.84 102.48) (width 0.25) (layer "F.Cu") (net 2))
 (segment (start 144.76 105.1) (end 144.84 105.02) (width 0.25) (layer "F.Cu") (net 2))
 (segment (start 138.2 99.85) (end 138.2 101.95) (width 0.25) (layer "F.Cu") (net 2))
 (segment (start 131.9 91.45) (end 131.9 101.95) (width 0.25) (layer "F.Cu") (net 2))
 (segment (start 123.5 95.65) (end 138.2 95.65) (width 0.25) (layer "F.Cu") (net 2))
 (segment (start 128.425 89.525) (end 133.275 89.525) (width 0.25) (layer "F.Cu") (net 2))
 (segment (start 129.8 91.45) (end 129.8 101.95) (width 0.25) (layer "F.Cu") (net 2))
 (segment (start 138.2 97.75) (end 123.5 97.75) (width 0.25) (layer "F.Cu") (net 2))
 (segment (start 124.025 89.525) (end 123.7 89.2) (width 0.25) (layer "F.Cu") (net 2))
 (segment (start 121.92 88.9) (end 123 88.9) (width 0.25) (layer "F.Cu") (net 2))
 (segment (start 124.326 80.534) (end 120.18 84.68) (width 0.25) (layer "F.Cu") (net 2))
 (segment (start 125.575 103.775) (end 125.9 104.1) (width 0.25) (layer "F.Cu") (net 2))
 (segment (start 123.5 88.4) (end 123.7 88.2) (width 0.25) (layer "F.Cu") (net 2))
 (segment (start 123.5 99.85) (end 138.2 99.85) (width 0.25) (layer "F.Cu") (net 2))
 (segment (start 138 105.1) (end 138 104.1) (width 0.25) (layer "F.Cu") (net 2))
 (segment (start 123.5 91.45) (end 123.5 93.55) (width 0.25) (layer "F.Cu") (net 2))
 (segment (start 116.94 105.1) (end 116.84 105) (width 0.25) (layer "F.Cu") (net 2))
 (segment (start 119.85 96.6) (end 120.85 96.6) (width 0.25) (layer "F.Cu") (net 2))
 (segment (start 128.3716 87.9284) (end 128.1 88.2) (width 0.25) (layer "F.Cu") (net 2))
 (segment (start 123.5 91.45) (end 123.5 88.4) (width 0.25) (layer "F.Cu") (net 2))
 (segment (start 136.1 91.45) (end 136.1 101.95) (width 0.25) (layer "F.Cu") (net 2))
 (segment (start 138.2 91.45) (end 138.2 93.55) (width 0.25) (layer "F.Cu") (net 2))
 (segment (start 131.9 91.45) (end 134 91.45) (width 0.25) (layer "F.Cu") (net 2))
 (segment (start 138.2 91.45) (end 138.2 101.95) (width 0.25) (layer "F.Cu") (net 2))
 (segment (start 123.5 91.45) (end 125.6 91.45) (width 0.25) (layer "F.Cu") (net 2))
 (segment (start 133.275 89.525) (end 133.6 89.2) (width 0.25) (layer "F.Cu") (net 2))
 (segment (start 133.6 89.2) (end 133.6 88.2) (width 0.25) (layer "F.Cu") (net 2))
 (segment (start 131.0212 80.534) (end 124.326 80.534) (width 0.25) (layer "F.Cu") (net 2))
 (segment (start 136.1 91.45) (end 138.2 91.45) (width 0.25) (layer "F.Cu") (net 2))
 (segment (start 123 88.9) (end 123.7 88.2) (width 0.25) (layer "F.Cu") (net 2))
 (segment (start 138 105.1) (end 142.24 105.1) (width 0.25) (layer "F.Cu") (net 2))
 (segment (start 128.1 88.2) (end 128.1 89.2) (width 0.25) (layer "F.Cu") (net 2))
 (segment (start 134 91.45) (end 134 101.95) (width 0.25) (layer "F.Cu") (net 2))
 (segment (start 129.8 91.45) (end 131.9 91.45) (width 0.25) (layer "F.Cu") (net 2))
 (segment (start 121.92 95.53) (end 121.92 88.9) (width 0.25) (layer "F.Cu") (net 2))
 (segment (start 142.24 105.1) (end 144.76 105.1) (width 0.25) (layer "F.Cu") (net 2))
 (segment (start 123.5 93.55) (end 123.5 95.65) (width 0.25) (layer "F.Cu") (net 2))
 (segment (start 120.85 96.6) (end 121.92 95.53) (width 0.25) (layer "F.Cu") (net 2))
 (segment (start 125.9 104.1) (end 125.9 105.1) (width 0.25) (layer "F.Cu") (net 2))
 (segment (start 123.7 89.2) (end 123.7 88.2) (width 0.25) (layer "F.Cu") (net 2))
 (segment (start 136.125 103.775) (end 135.8 104.1) (width 0.25) (layer "F.Cu") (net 2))
 (segment (start 123.7 88.2) (end 120.18 84.68) (width 0.25) (layer "F.Cu") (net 2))
 (segment (start 124.025 103.775) (end 125.575 103.775) (width 0.25) (layer "F.Cu") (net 2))
 (segment (start 123.5 95.65) (end 123.5 97.75) (width 0.25) (layer "F.Cu") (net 2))
 (segment (start 138.2 93.55) (end 123.5 93.55) (width 0.25) (layer "F.Cu") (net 2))
 (segment (start 132.5372 86.7156) (end 131.4196 86.7156) (width 0.25) (layer "F.Cu") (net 11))
 (segment (start 144.84 84.7) (end 144.84 82.1344) (width 0.25) (layer "F.Cu") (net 11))
 (segment (start 124.317801 85.2932) (end 124.3838 85.227201) (width 0.25) (layer "F.Cu") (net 11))
 (segment (start 131.4 86.7352) (end 131.4 88.2) (width 0.25) (layer "F.Cu") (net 11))
 (segment (start 144.84 84.7) (end 146.0844 84.7) (width 0.25) (layer "F.Cu") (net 11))
 (segment (start 131.4196 86.7156) (end 131.4 86.7352) (width 0.25) (layer "F.Cu") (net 11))
 (segment (start 132.5372 88.1628) (end 132.5 88.2) (width 0.25) (layer "F.Cu") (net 11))
 (segment (start 146.0844 84.7) (end 146.4564 84.328) (width 0.25) (layer "F.Cu") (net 11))
 (segment (start 122.7836 85.2932) (end 124.317801 85.2932) (width 0.25) (layer "F.Cu") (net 11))
 (segment (start 132.5372 86.7156) (end 132.5372 88.1628) (width 0.25) (layer "F.Cu") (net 11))
 (segment (start 146.4564 84.328) (end 146.4564 78.1304) (width 0.25) (layer "F.Cu") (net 11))
 (segment (start 144.84 82.1344) (end 144.8816 82.0928) (width 0.25) (layer "F.Cu") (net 11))
 (via (at 144.8816 82.0928) (size 0.8) (drill 0.4) (layers "F.Cu" "B.Cu") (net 11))
 (via (at 122.7836 85.2932) (size 0.8) (drill 0.4) (layers "F.Cu" "B.Cu") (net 11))
 (via (at 146.4564 78.1304) (size 0.8) (drill 0.4) (layers "F.Cu" "B.Cu") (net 11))
 (via (at 132.5372 86.7156) (size 0.8) (drill 0.4) (layers "F.Cu" "B.Cu") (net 11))
 (segment (start 125.0696 78.1304) (end 121.7168 81.4832) (width 0.25) (layer "B.Cu") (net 11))
 (segment (start 121.7168 85.1408) (end 121.666 85.1916) (width 0.25) (layer "B.Cu") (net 11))
 (segment (start 121.7168 81.4832) (end 121.7168 85.1408) (width 0.25) (layer "B.Cu") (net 11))
 (segment (start 121.666 85.1916) (end 122.682 85.1916) (width 0.25) (layer "B.Cu") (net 11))
 (segment (start 137.16 82.0928) (end 132.5372 86.7156) (width 0.25) (layer "B.Cu") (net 11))
 (segment (start 122.682 85.1916) (end 122.7836 85.2932) (width 0.25) (layer "B.Cu") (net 11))
 (segment (start 146.4564 78.1304) (end 125.0696 78.1304) (width 0.25) (layer "B.Cu") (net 11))
 (segment (start 144.8816 82.0928) (end 137.16 82.0928) (width 0.25) (layer "B.Cu") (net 11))
 (segment (start 130.3 105.1) (end 130.3 103.38) (width 0.25) (layer "F.Cu") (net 3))
 (segment (start 130.3 103.38) (end 130.3528 103.3272) (width 0.25) (layer "F.Cu") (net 3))
 (via (at 130.3528 103.3272) (size 0.8) (drill 0.4) (layers "F.Cu" "B.Cu") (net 3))
 (segment (start 117.7072 103.3272) (end 116.84 102.46) (width 0.25) (layer "B.Cu") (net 3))
 (segment (start 130.3528 103.3272) (end 117.7072 103.3272) (width 0.25) (layer "B.Cu") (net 3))
 (segment (start 119.85 102.1) (end 119.02 102.1) (width 0.25) (layer "F.Cu") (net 18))
 (segment (start 119.02 102.1) (end 116.84 99.92) (width 0.25) (layer "F.Cu") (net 18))
 (segment (start 118.85 99.9) (end 116.84 97.89) (width 0.25) (layer "F.Cu") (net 17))
 (segment (start 119.85 99.9) (end 118.85 99.9) (width 0.25) (layer "F.Cu") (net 17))
 (segment (start 116.84 97.89) (end 116.84 97.38) (width 0.25) (layer "F.Cu") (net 17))
 (segment (start 118.015 96.015) (end 116.84 94.84) (width 0.25) (layer "F.Cu") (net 16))
 (segment (start 118.015 97.965) (end 118.015 96.015) (width 0.25) (layer "F.Cu") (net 16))
 (segment (start 119.85 98.8) (end 118.85 98.8) (width 0.25) (layer "F.Cu") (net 16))
 (segment (start 118.85 98.8) (end 118.015 97.965) (width 0.25) (layer "F.Cu") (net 16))
 (segment (start 119.85 97.7) (end 118.85 97.7) (width 0.25) (layer "F.Cu") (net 15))
 (segment (start 118.85 97.7) (end 118.465 97.315) (width 0.25) (layer "F.Cu") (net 15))
 (segment (start 118.465 93.925) (end 116.84 92.3) (width 0.25) (layer "F.Cu") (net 15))
 (segment (start 118.465 97.315) (end 118.465 93.925) (width 0.25) (layer "F.Cu") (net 15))
 (segment (start 119.85 91.1) (end 118.18 91.1) (width 0.25) (layer "F.Cu") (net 14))
 (segment (start 118.18 91.1) (end 116.84 89.76) (width 0.25) (layer "F.Cu") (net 14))
 (segment (start 119.85 90) (end 117.07 87.22) (width 0.25) (layer "F.Cu") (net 13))
 (segment (start 117.07 87.22) (end 116.84 87.22) (width 0.25) (layer "F.Cu") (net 13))
 (segment (start 141.85 90) (end 144.61 87.24) (width 0.25) (layer "F.Cu") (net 10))
 (segment (start 144.61 87.24) (end 144.84 87.24) (width 0.25) (layer "F.Cu") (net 10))
 (segment (start 143.52 91.1) (end 144.84 89.78) (width 0.25) (layer "F.Cu") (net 9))
 (segment (start 141.85 91.1) (end 143.52 91.1) (width 0.25) (layer "F.Cu") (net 9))
 (segment (start 141.85 97.7) (end 140.85 97.7) (width 0.25) (layer "F.Cu") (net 8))
 (segment (start 143.215 99.535) (end 143.215 96.485) (width 0.25) (layer "F.Cu") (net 7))
 (segment (start 143.215 96.485) (end 144.84 94.86) (width 0.25) (layer "F.Cu") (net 7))
 (segment (start 142.85 99.9) (end 143.215 99.535) (width 0.25) (layer "F.Cu") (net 7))
 (segment (start 141.85 99.9) (end 142.85 99.9) (width 0.25) (layer "F.Cu") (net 7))
 (segment (start 141.85 101) (end 143.091701 101) (width 0.25) (layer "F.Cu") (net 6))
 (segment (start 143.091701 101) (end 143.665 100.426701) (width 0.25) (layer "F.Cu") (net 6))
 (segment (start 143.665 100.426701) (end 143.665 98.575) (width 0.25) (layer "F.Cu") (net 6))
 (segment (start 143.665 98.575) (end 144.84 97.4) (width 0.25) (layer "F.Cu") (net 6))
 (segment (start 142.68 102.1) (end 144.84 99.94) (width 0.25) (layer "F.Cu") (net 5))
 (segment (start 141.85 102.1) (end 142.68 102.1) (width 0.25) (layer "F.Cu") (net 5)))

